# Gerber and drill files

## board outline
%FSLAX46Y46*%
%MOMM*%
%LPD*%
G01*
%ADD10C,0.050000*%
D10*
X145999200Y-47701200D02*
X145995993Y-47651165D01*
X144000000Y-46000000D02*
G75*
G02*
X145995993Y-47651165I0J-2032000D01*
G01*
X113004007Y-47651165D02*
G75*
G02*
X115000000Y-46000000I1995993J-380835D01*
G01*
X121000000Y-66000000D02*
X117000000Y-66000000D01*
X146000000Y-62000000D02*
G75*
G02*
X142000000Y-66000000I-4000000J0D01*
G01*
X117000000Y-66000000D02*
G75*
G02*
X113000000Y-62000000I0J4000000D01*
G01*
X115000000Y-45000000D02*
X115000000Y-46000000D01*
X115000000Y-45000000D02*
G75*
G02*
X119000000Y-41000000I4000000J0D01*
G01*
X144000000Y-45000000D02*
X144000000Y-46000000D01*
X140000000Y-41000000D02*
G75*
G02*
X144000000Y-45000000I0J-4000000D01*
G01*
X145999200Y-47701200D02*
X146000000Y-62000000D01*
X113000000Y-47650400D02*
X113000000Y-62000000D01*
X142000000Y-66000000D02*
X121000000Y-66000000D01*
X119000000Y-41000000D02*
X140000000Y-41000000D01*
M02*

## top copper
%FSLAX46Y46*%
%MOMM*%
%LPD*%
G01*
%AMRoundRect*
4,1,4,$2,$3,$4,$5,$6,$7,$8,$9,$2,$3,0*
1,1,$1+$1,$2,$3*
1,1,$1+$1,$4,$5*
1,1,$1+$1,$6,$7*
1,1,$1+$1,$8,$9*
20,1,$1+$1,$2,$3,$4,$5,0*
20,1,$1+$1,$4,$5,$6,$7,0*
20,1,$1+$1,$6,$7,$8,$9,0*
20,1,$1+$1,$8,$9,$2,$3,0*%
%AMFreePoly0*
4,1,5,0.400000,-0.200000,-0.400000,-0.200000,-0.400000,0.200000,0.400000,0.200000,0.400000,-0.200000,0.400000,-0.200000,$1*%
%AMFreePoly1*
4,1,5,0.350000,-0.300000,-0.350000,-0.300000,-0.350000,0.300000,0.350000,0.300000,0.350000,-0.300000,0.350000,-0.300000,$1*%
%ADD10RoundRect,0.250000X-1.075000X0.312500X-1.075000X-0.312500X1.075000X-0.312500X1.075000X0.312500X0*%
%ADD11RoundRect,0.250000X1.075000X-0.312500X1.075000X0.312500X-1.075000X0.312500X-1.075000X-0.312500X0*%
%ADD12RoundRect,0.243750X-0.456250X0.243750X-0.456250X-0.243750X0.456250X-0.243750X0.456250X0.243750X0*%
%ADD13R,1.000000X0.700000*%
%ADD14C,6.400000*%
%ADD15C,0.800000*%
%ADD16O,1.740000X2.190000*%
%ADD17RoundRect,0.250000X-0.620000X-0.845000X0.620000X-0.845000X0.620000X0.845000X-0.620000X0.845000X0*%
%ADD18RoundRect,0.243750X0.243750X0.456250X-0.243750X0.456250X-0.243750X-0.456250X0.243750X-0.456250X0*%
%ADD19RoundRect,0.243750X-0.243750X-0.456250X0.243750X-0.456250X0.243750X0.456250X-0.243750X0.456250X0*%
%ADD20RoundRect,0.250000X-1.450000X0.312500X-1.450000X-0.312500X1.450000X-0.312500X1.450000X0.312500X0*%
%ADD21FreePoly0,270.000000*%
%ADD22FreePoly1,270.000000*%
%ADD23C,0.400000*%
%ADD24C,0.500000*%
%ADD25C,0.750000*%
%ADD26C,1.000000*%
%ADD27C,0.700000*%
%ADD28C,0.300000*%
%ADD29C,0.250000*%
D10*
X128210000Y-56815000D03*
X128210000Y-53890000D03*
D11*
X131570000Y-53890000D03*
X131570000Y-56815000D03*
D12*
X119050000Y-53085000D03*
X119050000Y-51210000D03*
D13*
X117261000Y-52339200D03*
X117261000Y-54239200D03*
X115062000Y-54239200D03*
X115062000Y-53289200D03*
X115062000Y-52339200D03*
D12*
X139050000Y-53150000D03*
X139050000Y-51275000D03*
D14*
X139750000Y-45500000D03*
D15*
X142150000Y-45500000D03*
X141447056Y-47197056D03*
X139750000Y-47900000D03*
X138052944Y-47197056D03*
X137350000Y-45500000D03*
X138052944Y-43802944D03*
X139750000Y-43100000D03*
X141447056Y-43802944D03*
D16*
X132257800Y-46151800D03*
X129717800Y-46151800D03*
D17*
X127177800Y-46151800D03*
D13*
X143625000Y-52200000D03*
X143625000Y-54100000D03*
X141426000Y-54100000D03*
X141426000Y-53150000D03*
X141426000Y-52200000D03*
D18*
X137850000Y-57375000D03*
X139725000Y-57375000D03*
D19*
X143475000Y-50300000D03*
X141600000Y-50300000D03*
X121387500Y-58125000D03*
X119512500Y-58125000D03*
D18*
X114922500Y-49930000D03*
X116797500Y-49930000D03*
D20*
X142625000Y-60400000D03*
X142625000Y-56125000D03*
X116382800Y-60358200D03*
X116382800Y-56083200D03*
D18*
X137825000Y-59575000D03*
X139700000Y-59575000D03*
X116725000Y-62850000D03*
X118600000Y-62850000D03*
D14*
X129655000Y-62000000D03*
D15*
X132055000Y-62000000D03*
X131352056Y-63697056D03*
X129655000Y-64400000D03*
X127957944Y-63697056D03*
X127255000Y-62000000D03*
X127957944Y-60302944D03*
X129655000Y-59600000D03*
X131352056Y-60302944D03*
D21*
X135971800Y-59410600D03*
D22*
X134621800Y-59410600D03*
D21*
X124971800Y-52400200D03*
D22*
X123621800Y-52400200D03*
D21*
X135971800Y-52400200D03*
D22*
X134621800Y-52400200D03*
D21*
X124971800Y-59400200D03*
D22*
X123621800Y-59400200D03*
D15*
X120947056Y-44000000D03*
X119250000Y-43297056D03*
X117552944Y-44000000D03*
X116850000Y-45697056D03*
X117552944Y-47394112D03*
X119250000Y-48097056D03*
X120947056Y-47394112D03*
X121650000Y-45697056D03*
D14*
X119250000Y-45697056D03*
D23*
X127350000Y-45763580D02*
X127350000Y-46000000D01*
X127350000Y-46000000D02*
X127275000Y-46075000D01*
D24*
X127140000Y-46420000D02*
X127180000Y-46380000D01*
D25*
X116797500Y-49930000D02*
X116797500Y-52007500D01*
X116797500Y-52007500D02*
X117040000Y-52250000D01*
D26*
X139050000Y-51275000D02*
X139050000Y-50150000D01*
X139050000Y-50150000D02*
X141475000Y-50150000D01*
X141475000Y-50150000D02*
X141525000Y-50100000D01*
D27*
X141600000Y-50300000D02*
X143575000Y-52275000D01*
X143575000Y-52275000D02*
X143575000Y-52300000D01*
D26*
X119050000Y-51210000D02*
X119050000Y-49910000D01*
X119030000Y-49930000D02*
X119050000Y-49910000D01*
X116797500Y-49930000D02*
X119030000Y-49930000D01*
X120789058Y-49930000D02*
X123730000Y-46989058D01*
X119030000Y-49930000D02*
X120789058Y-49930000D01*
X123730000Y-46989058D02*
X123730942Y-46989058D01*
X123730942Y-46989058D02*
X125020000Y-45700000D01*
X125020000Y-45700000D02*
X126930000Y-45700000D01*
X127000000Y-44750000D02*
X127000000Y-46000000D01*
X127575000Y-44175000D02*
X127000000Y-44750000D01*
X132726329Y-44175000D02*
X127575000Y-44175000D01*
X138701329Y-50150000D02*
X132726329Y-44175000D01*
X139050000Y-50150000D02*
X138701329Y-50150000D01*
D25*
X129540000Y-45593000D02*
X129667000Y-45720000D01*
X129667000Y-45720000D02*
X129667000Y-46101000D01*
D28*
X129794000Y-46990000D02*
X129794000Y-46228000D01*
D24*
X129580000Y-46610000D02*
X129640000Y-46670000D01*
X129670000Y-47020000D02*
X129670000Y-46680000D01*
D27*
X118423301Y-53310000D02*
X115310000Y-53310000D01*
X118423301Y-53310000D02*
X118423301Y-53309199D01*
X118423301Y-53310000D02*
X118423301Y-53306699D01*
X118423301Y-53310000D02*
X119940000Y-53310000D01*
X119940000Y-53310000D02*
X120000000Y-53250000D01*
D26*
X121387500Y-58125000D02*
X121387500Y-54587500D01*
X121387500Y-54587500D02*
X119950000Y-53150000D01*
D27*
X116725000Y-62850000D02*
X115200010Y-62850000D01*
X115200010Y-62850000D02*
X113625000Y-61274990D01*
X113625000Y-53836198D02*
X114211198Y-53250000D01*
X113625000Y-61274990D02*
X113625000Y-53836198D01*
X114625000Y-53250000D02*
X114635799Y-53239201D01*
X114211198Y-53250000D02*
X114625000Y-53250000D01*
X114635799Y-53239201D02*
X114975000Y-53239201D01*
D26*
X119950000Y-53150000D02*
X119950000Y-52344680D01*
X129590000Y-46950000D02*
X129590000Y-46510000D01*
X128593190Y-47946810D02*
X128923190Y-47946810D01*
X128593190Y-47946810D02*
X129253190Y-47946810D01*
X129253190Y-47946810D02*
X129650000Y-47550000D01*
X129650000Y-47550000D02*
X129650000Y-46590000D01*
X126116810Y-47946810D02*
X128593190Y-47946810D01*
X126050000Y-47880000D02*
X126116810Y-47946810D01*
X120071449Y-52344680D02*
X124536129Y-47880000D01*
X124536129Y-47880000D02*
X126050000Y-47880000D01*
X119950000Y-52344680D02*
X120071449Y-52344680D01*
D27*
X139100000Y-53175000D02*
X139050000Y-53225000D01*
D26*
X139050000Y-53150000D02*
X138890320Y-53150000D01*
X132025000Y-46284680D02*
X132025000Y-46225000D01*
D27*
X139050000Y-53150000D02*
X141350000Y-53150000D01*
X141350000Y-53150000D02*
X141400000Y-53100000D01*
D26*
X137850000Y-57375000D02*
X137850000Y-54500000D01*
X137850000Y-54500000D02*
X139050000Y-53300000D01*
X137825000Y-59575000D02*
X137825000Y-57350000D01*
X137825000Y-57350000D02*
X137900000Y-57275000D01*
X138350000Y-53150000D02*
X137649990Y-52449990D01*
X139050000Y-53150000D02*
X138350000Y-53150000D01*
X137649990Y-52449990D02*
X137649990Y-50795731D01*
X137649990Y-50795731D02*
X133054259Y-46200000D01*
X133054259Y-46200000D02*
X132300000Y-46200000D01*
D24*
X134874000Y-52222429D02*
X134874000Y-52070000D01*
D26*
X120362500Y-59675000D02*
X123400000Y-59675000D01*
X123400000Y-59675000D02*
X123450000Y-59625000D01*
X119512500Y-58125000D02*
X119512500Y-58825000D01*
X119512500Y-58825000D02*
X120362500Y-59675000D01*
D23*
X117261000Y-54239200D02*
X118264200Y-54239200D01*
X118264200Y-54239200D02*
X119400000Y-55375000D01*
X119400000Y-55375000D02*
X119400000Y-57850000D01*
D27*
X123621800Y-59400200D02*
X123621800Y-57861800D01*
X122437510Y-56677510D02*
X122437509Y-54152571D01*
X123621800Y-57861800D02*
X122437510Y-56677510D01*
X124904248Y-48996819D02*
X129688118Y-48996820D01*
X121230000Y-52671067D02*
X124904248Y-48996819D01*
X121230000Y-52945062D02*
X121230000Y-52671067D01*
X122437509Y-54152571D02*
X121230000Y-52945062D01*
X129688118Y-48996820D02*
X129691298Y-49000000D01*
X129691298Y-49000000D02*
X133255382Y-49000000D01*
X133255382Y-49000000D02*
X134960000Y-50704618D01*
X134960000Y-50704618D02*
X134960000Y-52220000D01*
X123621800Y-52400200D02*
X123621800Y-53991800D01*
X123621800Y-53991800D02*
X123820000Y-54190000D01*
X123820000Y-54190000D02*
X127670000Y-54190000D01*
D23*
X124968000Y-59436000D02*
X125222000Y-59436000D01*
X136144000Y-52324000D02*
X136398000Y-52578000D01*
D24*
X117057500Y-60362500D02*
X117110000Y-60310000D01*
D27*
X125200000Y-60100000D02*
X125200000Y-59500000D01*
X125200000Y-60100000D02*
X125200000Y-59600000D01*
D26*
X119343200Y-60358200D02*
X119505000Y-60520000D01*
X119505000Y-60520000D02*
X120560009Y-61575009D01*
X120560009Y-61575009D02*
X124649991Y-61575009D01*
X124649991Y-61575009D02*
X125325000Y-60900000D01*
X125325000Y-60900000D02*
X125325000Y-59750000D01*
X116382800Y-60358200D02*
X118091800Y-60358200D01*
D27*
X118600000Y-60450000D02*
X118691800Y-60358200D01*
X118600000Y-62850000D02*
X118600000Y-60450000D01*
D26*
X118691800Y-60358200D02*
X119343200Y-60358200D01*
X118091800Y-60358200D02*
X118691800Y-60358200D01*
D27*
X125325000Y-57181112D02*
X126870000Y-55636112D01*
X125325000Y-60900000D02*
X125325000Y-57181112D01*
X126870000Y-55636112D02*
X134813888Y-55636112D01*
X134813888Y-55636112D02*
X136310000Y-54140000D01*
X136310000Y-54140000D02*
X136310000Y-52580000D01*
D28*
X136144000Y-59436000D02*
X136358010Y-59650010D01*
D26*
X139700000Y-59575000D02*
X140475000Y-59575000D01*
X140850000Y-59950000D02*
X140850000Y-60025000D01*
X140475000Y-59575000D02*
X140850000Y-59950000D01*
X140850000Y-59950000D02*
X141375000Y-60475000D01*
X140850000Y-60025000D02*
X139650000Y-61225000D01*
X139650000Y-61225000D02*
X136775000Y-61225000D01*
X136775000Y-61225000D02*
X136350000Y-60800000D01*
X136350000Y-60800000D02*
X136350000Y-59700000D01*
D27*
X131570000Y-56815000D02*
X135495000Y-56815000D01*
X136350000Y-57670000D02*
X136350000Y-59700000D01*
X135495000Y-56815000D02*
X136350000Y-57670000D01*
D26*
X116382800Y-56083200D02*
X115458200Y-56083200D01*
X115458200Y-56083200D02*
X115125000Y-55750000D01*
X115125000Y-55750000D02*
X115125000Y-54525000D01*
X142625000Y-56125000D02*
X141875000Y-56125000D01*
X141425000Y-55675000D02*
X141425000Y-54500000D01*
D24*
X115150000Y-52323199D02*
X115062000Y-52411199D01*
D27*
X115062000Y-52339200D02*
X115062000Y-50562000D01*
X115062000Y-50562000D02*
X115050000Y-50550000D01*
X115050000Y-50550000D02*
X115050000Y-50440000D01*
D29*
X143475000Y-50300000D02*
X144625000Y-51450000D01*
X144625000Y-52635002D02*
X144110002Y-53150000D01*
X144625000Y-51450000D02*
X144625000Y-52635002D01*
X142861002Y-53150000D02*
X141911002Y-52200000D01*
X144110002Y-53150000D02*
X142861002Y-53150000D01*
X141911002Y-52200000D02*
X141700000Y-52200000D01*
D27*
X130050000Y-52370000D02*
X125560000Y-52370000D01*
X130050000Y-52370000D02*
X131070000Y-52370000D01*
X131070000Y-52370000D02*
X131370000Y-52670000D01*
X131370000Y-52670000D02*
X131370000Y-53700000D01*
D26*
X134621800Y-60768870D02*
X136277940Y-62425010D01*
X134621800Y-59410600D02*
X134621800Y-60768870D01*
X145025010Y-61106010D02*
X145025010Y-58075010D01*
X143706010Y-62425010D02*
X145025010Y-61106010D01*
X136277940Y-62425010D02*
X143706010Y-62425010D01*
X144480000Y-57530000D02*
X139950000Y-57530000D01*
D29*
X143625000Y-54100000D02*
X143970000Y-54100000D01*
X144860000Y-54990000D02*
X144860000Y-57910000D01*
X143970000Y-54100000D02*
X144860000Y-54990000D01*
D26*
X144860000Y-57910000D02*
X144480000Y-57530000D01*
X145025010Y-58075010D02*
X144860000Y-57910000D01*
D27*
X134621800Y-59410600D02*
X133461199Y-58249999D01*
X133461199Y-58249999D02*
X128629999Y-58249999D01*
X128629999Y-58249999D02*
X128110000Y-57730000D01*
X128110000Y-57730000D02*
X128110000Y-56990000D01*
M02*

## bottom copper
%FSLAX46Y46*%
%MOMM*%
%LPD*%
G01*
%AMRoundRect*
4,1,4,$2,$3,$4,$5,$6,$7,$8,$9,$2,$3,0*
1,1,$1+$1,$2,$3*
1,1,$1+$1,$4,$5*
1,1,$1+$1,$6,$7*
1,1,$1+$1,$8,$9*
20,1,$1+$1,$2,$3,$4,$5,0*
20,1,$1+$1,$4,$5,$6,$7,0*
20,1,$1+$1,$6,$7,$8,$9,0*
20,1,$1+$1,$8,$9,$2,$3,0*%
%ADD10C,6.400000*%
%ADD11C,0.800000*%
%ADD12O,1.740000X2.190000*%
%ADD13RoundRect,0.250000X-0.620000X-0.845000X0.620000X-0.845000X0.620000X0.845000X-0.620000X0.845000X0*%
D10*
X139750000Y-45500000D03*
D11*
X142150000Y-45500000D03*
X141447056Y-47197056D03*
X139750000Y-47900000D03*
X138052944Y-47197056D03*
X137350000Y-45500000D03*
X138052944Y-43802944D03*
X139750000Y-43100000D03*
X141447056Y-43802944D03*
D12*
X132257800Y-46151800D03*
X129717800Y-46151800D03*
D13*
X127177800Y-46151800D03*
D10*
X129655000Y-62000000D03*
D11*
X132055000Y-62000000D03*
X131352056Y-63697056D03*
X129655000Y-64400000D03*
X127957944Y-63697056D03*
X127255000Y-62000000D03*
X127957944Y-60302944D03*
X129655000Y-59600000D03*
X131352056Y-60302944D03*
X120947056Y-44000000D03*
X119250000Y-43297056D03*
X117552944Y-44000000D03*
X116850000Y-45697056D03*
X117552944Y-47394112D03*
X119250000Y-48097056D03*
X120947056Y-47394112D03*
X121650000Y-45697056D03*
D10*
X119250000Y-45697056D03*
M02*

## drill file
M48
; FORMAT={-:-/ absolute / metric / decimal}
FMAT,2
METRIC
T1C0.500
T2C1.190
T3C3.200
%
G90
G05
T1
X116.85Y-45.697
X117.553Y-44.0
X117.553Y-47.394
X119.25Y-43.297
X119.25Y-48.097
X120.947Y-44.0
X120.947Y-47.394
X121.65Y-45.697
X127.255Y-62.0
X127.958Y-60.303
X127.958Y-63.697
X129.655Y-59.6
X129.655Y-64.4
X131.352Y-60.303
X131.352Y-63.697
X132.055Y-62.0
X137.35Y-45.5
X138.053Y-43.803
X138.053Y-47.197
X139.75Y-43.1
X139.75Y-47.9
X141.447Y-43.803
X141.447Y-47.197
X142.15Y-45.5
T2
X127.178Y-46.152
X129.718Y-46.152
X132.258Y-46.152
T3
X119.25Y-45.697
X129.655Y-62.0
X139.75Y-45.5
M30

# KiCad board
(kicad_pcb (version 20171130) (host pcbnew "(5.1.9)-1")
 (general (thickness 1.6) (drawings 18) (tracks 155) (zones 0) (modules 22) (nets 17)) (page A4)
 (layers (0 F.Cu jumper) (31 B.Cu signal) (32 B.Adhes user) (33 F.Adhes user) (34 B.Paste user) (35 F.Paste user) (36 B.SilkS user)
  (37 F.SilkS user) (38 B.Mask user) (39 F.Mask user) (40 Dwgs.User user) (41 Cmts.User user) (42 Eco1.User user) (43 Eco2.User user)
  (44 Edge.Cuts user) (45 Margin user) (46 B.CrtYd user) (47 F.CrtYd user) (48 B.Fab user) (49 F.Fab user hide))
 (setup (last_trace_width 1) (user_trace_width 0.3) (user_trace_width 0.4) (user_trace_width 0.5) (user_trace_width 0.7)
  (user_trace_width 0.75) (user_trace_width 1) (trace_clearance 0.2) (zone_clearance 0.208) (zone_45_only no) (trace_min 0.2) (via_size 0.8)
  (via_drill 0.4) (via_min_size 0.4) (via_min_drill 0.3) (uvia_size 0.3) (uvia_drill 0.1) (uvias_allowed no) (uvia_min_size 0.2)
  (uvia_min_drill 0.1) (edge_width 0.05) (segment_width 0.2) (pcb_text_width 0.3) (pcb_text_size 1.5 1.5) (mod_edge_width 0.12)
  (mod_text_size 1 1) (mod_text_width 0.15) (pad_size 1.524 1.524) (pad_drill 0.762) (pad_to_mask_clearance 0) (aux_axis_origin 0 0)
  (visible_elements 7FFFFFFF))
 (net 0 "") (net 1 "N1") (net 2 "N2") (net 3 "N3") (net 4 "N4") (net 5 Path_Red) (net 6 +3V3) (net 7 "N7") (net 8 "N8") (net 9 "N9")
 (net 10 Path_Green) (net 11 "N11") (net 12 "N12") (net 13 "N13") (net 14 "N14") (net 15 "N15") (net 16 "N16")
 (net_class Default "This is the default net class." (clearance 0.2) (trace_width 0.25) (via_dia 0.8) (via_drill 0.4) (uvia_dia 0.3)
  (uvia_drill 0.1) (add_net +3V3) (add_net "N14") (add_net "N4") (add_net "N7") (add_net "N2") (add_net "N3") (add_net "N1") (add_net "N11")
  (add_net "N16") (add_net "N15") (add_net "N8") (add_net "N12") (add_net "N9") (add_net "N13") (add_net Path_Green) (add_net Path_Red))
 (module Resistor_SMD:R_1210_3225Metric (layer F.Cu) (at 128.21 55.3525 270)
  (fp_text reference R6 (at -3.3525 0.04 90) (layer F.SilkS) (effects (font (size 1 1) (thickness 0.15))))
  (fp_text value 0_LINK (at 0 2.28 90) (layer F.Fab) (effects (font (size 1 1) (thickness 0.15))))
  (pad 2 smd roundrect (at 1.4625 0 270) (size 1.125 2.65) (layers F.Cu F.Paste F.Mask) (roundrect_rratio 0.222222) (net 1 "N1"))
  (pad 1 smd roundrect (at -1.4625 0 270) (size 1.125 2.65) (layers F.Cu F.Paste F.Mask) (roundrect_rratio 0.222222) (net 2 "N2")))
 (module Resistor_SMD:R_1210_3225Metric (layer F.Cu) (at 131.57 55.3525 90)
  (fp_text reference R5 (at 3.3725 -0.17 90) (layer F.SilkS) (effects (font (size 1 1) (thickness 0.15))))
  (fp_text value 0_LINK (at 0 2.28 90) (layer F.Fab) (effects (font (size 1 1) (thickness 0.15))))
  (pad 2 smd roundrect (at 1.4625 0 90) (size 1.125 2.65) (layers F.Cu F.Paste F.Mask) (roundrect_rratio 0.222222) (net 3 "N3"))
  (pad 1 smd roundrect (at -1.4625 0 90) (size 1.125 2.65) (layers F.Cu F.Paste F.Mask) (roundrect_rratio 0.222222) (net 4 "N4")))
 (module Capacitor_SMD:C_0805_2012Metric (layer F.Cu) (at 119.05 52.1475 270)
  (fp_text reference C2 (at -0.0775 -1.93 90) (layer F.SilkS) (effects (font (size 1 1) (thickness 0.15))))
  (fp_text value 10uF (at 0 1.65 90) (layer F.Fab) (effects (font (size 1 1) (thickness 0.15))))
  (pad 2 smd roundrect (at 0.9375 0 270) (size 0.975 1.4) (layers F.Cu F.Paste F.Mask) (roundrect_rratio 0.25) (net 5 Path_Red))
  (pad 1 smd roundrect (at -0.9375 0 270) (size 0.975 1.4) (layers F.Cu F.Paste F.Mask) (roundrect_rratio 0.25) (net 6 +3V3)))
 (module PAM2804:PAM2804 (layer F.Cu) (at 115.062 52.3392)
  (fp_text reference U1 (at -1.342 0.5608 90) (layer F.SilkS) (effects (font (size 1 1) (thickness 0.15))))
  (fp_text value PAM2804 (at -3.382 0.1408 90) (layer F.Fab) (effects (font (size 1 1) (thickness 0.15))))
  (pad 5 smd rect (at 2.199 0) (size 1 0.7) (layers F.Cu F.Paste F.Mask) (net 6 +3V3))
  (pad 4 smd rect (at 2.199 1.9) (size 1 0.7) (layers F.Cu F.Paste F.Mask) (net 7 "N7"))
  (pad 3 smd rect (at 0 1.9) (size 1 0.7) (layers F.Cu F.Paste F.Mask) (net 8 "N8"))
  (pad 2 smd rect (at 0 0.95) (size 1 0.7) (layers F.Cu F.Paste F.Mask) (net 5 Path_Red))
  (pad 1 smd rect (at 0 0) (size 1 0.7) (layers F.Cu F.Paste F.Mask) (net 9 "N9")))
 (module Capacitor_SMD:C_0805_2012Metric (layer F.Cu) (at 139.05 52.2125 270)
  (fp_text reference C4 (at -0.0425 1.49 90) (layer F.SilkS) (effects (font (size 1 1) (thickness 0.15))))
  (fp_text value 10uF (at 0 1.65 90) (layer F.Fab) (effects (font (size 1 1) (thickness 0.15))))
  (pad 2 smd roundrect (at 0.9375 0 270) (size 0.975 1.4) (layers F.Cu F.Paste F.Mask) (roundrect_rratio 0.25) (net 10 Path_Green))
  (pad 1 smd roundrect (at -0.9375 0 270) (size 0.975 1.4) (layers F.Cu F.Paste F.Mask) (roundrect_rratio 0.25) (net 6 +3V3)))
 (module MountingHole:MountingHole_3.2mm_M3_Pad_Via (layer F.Cu) (at 139.75 45.5)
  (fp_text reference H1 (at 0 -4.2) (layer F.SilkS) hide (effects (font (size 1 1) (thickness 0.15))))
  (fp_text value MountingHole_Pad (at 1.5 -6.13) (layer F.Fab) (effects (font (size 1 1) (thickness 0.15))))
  (pad 1 thru_hole circle (at 0 0) (size 6.4 6.4) (drill 3.2) (layers *.Cu *.Mask) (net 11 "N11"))
  (pad 1 thru_hole circle (at 2.4 0) (size 0.8 0.8) (drill 0.5) (layers *.Cu *.Mask) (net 11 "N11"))
  (pad 1 thru_hole circle (at 1.697056 1.697056) (size 0.8 0.8) (drill 0.5) (layers *.Cu *.Mask) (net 11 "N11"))
  (pad 1 thru_hole circle (at 0 2.4) (size 0.8 0.8) (drill 0.5) (layers *.Cu *.Mask) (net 11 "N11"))
  (pad 1 thru_hole circle (at -1.697056 1.697056) (size 0.8 0.8) (drill 0.5) (layers *.Cu *.Mask) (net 11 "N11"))
  (pad 1 thru_hole circle (at -2.4 0) (size 0.8 0.8) (drill 0.5) (layers *.Cu *.Mask) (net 11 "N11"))
  (pad 1 thru_hole circle (at -1.697056 -1.697056) (size 0.8 0.8) (drill 0.5) (layers *.Cu *.Mask) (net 11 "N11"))
  (pad 1 thru_hole circle (at 0 -2.4) (size 0.8 0.8) (drill 0.5) (layers *.Cu *.Mask) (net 11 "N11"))
  (pad 1 thru_hole circle (at 1.697056 -1.697056) (size 0.8 0.8) (drill 0.5) (layers *.Cu *.Mask) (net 11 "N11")))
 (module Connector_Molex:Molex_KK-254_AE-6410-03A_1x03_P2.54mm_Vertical (layer F.Cu) (at 127.1778 46.1518)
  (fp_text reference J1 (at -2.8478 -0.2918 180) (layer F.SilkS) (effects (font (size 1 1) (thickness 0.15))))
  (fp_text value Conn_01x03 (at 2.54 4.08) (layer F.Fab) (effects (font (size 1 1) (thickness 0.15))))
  (pad 3 thru_hole oval (at 5.08 0) (size 1.74 2.19) (drill 1.19) (layers *.Cu *.Mask) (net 10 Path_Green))
  (pad 2 thru_hole oval (at 2.54 0) (size 1.74 2.19) (drill 1.19) (layers *.Cu *.Mask) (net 5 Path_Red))
  (pad 1 thru_hole roundrect (at 0 0) (size 1.74 2.19) (drill 1.19) (layers *.Cu *.Mask) (roundrect_rratio 0.143678) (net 6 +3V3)))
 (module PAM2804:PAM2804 (layer F.Cu) (at 141.426 52.2)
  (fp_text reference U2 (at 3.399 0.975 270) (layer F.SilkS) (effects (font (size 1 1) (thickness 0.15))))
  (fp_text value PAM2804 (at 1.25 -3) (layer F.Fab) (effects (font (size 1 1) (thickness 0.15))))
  (pad 5 smd rect (at 2.199 0) (size 1 0.7) (layers F.Cu F.Paste F.Mask) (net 6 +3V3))
  (pad 4 smd rect (at 2.199 1.9) (size 1 0.7) (layers F.Cu F.Paste F.Mask) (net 1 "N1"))
  (pad 3 smd rect (at 0 1.9) (size 1 0.7) (layers F.Cu F.Paste F.Mask) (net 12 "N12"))
  (pad 2 smd rect (at 0 0.95) (size 1 0.7) (layers F.Cu F.Paste F.Mask) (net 10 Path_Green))
  (pad 1 smd rect (at 0 0) (size 1 0.7) (layers F.Cu F.Paste F.Mask) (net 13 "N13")))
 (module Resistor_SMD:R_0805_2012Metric (layer F.Cu) (at 138.7875 57.375 180)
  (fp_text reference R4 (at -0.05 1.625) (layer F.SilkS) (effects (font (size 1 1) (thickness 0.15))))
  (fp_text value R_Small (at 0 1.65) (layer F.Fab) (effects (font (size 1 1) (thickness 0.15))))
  (pad 2 smd roundrect (at 0.9375 0 180) (size 0.975 1.4) (layers F.Cu F.Paste F.Mask) (roundrect_rratio 0.25) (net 10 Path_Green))
  (pad 1 smd roundrect (at -0.9375 0 180) (size 0.975 1.4) (layers F.Cu F.Paste F.Mask) (roundrect_rratio 0.25) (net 1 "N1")))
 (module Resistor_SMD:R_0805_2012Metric (layer F.Cu) (at 142.5375 50.3)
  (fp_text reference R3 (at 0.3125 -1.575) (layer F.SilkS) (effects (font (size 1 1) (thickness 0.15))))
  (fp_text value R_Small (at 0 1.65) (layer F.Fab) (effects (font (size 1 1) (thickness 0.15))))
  (pad 2 smd roundrect (at 0.9375 0) (size 0.975 1.4) (layers F.Cu F.Paste F.Mask) (roundrect_rratio 0.25) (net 13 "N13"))
  (pad 1 smd roundrect (at -0.9375 0) (size 0.975 1.4) (layers F.Cu F.Paste F.Mask) (roundrect_rratio 0.25) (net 6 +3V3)))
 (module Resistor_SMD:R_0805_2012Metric (layer F.Cu) (at 120.45 58.125)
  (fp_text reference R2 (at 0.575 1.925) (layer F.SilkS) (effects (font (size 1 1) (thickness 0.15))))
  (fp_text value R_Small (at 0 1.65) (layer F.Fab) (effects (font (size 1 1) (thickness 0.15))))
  (pad 2 smd roundrect (at 0.9375 0) (size 0.975 1.4) (layers F.Cu F.Paste F.Mask) (roundrect_rratio 0.25) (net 5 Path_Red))
  (pad 1 smd roundrect (at -0.9375 0) (size 0.975 1.4) (layers F.Cu F.Paste F.Mask) (roundrect_rratio 0.25) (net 7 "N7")))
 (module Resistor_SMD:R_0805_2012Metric (layer F.Cu) (at 115.86 49.93 180)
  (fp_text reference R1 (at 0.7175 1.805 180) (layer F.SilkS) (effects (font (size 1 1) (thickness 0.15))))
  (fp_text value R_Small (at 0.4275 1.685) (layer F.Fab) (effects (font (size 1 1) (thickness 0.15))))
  (pad 2 smd roundrect (at 0.9375 0 180) (size 0.975 1.4) (layers F.Cu F.Paste F.Mask) (roundrect_rratio 0.25) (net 9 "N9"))
  (pad 1 smd roundrect (at -0.9375 0 180) (size 0.975 1.4) (layers F.Cu F.Paste F.Mask) (roundrect_rratio 0.25) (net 6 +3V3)))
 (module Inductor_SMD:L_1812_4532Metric (layer F.Cu) (at 142.625 58.2625 270)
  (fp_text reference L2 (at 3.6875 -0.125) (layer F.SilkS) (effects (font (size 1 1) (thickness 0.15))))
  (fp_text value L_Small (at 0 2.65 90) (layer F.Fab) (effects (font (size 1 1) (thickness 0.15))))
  (pad 2 smd roundrect (at 2.1375 0 270) (size 1.125 3.4) (layers F.Cu F.Paste F.Mask) (roundrect_rratio 0.222222) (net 4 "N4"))
  (pad 1 smd roundrect (at -2.1375 0 270) (size 1.125 3.4) (layers F.Cu F.Paste F.Mask) (roundrect_rratio 0.222222) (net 12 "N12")))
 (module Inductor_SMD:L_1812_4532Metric (layer F.Cu) (at 116.3828 58.2207 270)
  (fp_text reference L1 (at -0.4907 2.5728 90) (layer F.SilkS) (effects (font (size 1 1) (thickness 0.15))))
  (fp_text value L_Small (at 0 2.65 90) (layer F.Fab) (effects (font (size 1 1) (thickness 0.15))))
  (pad 2 smd roundrect (at 2.1375 0 270) (size 1.125 3.4) (layers F.Cu F.Paste F.Mask) (roundrect_rratio 0.222222) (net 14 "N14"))
  (pad 1 smd roundrect (at -2.1375 0 270) (size 1.125 3.4) (layers F.Cu F.Paste F.Mask) (roundrect_rratio 0.222222) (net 8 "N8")))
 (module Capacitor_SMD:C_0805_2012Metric (layer F.Cu) (at 138.7625 59.575 180)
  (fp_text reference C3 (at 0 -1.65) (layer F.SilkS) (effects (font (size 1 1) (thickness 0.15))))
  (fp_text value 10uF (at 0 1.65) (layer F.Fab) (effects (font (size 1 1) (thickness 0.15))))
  (pad 2 smd roundrect (at 0.9375 0 180) (size 0.975 1.4) (layers F.Cu F.Paste F.Mask) (roundrect_rratio 0.25) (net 10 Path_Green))
  (pad 1 smd roundrect (at -0.9375 0 180) (size 0.975 1.4) (layers F.Cu F.Paste F.Mask) (roundrect_rratio 0.25) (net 4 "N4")))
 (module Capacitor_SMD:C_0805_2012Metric (layer F.Cu) (at 117.6625 62.85 180)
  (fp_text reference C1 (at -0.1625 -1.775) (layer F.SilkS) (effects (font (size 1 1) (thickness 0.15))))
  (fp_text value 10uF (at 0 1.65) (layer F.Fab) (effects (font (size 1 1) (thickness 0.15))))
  (pad 2 smd roundrect (at 0.9375 0 180) (size 0.975 1.4) (layers F.Cu F.Paste F.Mask) (roundrect_rratio 0.25) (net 5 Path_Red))
  (pad 1 smd roundrect (at -0.9375 0 180) (size 0.975 1.4) (layers F.Cu F.Paste F.Mask) (roundrect_rratio 0.25) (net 14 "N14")))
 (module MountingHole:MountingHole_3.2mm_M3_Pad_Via (layer F.Cu) (at 129.655 62)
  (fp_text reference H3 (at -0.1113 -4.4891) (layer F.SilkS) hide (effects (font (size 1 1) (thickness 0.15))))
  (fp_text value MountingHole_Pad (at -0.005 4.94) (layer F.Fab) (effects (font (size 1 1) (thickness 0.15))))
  (pad 1 thru_hole circle (at 0 0) (size 6.4 6.4) (drill 3.2) (layers *.Cu *.Mask) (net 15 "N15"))
  (pad 1 thru_hole circle (at 2.4 0) (size 0.8 0.8) (drill 0.5) (layers *.Cu *.Mask) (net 15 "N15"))
  (pad 1 thru_hole circle (at 1.697056 1.697056) (size 0.8 0.8) (drill 0.5) (layers *.Cu *.Mask) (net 15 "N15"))
  (pad 1 thru_hole circle (at 0 2.4) (size 0.8 0.8) (drill 0.5) (layers *.Cu *.Mask) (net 15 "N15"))
  (pad 1 thru_hole circle (at -1.697056 1.697056) (size 0.8 0.8) (drill 0.5) (layers *.Cu *.Mask) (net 15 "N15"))
  (pad 1 thru_hole circle (at -2.4 0) (size 0.8 0.8) (drill 0.5) (layers *.Cu *.Mask) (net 15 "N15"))
  (pad 1 thru_hole circle (at -1.697056 -1.697056) (size 0.8 0.8) (drill 0.5) (layers *.Cu *.Mask) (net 15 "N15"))
  (pad 1 thru_hole circle (at 0 -2.4) (size 0.8 0.8) (drill 0.5) (layers *.Cu *.Mask) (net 15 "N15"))
  (pad 1 thru_hole circle (at 1.697056 -1.697056) (size 0.8 0.8) (drill 0.5) (layers *.Cu *.Mask) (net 15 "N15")))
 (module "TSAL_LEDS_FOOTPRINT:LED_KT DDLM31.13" (layer F.Cu) (at 135.2468 59.3856 270)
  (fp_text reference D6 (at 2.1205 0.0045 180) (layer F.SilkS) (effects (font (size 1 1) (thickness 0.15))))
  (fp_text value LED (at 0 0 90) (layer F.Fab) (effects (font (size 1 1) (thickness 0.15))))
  (pad 2 smd custom (at 0.025 -0.725 270) (size 0.8 0.4) (layers F.Cu F.Paste F.Mask) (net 4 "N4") (zone_connect 0)
   (options (clearance outline) (anchor rect)) (primitives))
  (pad 1 smd custom (at 0.025 0.625 270) (size 0.7 0.6) (layers F.Cu F.Paste F.Mask) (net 1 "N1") (zone_connect 0)
   (options (clearance outline) (anchor rect)) (primitives)))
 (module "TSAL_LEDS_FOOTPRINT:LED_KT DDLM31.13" (layer F.Cu) (at 124.2468 52.3752 270)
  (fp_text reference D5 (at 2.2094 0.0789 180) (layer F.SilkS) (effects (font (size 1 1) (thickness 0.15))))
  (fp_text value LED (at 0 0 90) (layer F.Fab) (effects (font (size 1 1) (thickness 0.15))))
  (pad 2 smd custom (at 0.025 -0.725 270) (size 0.8 0.4) (layers F.Cu F.Paste F.Mask) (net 3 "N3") (zone_connect 0)
   (options (clearance outline) (anchor rect)) (primitives))
  (pad 1 smd custom (at 0.025 0.625 270) (size 0.7 0.6) (layers F.Cu F.Paste F.Mask) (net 2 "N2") (zone_connect 0)
   (options (clearance outline) (anchor rect)) (primitives)))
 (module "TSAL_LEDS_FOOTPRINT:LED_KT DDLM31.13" (layer F.Cu) (at 135.2468 52.3752 270)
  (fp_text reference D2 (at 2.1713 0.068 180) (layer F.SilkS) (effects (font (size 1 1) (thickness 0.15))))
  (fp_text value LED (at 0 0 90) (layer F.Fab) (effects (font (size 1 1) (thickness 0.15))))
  (pad 2 smd custom (at 0.025 -0.725 270) (size 0.8 0.4) (layers F.Cu F.Paste F.Mask) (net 14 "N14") (zone_connect 0)
   (options (clearance outline) (anchor rect)) (primitives))
  (pad 1 smd custom (at 0.025 0.625 270) (size 0.7 0.6) (layers F.Cu F.Paste F.Mask) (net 7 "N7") (zone_connect 0)
   (options (clearance outline) (anchor rect)) (primitives)))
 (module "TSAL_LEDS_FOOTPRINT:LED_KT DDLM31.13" (layer F.Cu) (at 124.2468 59.3752 270)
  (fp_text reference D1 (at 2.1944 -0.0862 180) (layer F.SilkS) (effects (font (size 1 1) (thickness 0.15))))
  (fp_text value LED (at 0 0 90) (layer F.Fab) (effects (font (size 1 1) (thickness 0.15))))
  (pad 2 smd custom (at 0.025 -0.725 270) (size 0.8 0.4) (layers F.Cu F.Paste F.Mask) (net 14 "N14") (zone_connect 0)
   (options (clearance outline) (anchor rect)) (primitives))
  (pad 1 smd custom (at 0.025 0.625 270) (size 0.7 0.6) (layers F.Cu F.Paste F.Mask) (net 7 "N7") (zone_connect 0)
   (options (clearance outline) (anchor rect)) (primitives)))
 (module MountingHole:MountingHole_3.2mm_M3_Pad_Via (layer F.Cu) (at 119.25 45.697056)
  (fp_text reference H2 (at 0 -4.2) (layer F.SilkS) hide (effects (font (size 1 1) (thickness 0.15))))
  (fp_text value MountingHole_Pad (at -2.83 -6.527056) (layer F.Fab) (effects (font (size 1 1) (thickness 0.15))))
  (pad 1 thru_hole circle (at 1.697056 -1.697056) (size 0.8 0.8) (drill 0.5) (layers *.Cu *.Mask) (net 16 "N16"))
  (pad 1 thru_hole circle (at 0 -2.4) (size 0.8 0.8) (drill 0.5) (layers *.Cu *.Mask) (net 16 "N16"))
  (pad 1 thru_hole circle (at -1.697056 -1.697056) (size 0.8 0.8) (drill 0.5) (layers *.Cu *.Mask) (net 16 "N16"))
  (pad 1 thru_hole circle (at -2.4 0) (size 0.8 0.8) (drill 0.5) (layers *.Cu *.Mask) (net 16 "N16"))
  (pad 1 thru_hole circle (at -1.697056 1.697056) (size 0.8 0.8) (drill 0.5) (layers *.Cu *.Mask) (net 16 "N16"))
  (pad 1 thru_hole circle (at 0 2.4) (size 0.8 0.8) (drill 0.5) (layers *.Cu *.Mask) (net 16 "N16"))
  (pad 1 thru_hole circle (at 1.697056 1.697056) (size 0.8 0.8) (drill 0.5) (layers *.Cu *.Mask) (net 16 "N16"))
  (pad 1 thru_hole circle (at 2.4 0) (size 0.8 0.8) (drill 0.5) (layers *.Cu *.Mask) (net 16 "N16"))
  (pad 1 thru_hole circle (at 0 0) (size 6.4 6.4) (drill 3.2) (layers *.Cu *.Mask) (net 16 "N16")))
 (gr_line (start 145.9992 47.7012) (end 145.995993 47.651165) (layer Edge.Cuts) (width 0.05))
 (gr_arc (start 144 48.032) (end 144 46) (angle 79.1978127) (layer Edge.Cuts) (width 0.05))
 (gr_arc (start 115 48.032) (end 115 46) (angle -79.1978127) (layer Edge.Cuts) (width 0.05))
 (gr_line (start 121 66) (end 117 66) (layer Edge.Cuts) (width 0.05))
 (gr_arc (start 142 62) (end 142 66) (angle -90) (layer Edge.Cuts) (width 0.05))
 (gr_arc (start 117 62) (end 113 62) (angle -90) (layer Edge.Cuts) (width 0.05))
 (gr_line (start 115 45) (end 115 46) (layer Edge.Cuts) (width 0.05))
 (gr_arc (start 119 45) (end 119 41) (angle -90) (layer Edge.Cuts) (width 0.05))
 (gr_line (start 144 45) (end 144 46) (layer Edge.Cuts) (width 0.05))
 (gr_arc (start 140 45) (end 144 45) (angle -90) (layer Edge.Cuts) (width 0.05))
 (gr_line (start 145.9992 47.7012) (end 146 62) (layer Edge.Cuts) (width 0.05))
 (gr_line (start 113 47.6504) (end 113 62) (layer Edge.Cuts) (width 0.05))
 (gr_line (start 142 66) (end 121 66) (layer Edge.Cuts) (width 0.05))
 (gr_line (start 119 41) (end 140 41) (layer Edge.Cuts) (width 0.05))
 (segment (start 127.35 45.76358) (end 127.35 46) (width 0.4) (layer F.Cu) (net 6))
 (segment (start 127.35 46) (end 127.275 46.075) (width 0.4) (layer F.Cu) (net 6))
 (segment (start 127.14 46.42) (end 127.18 46.38) (width 0.5) (layer F.Cu) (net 6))
 (segment (start 116.7975 49.93) (end 116.7975 52.0075) (width 0.75) (layer F.Cu) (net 6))
 (segment (start 116.7975 52.0075) (end 117.04 52.25) (width 0.75) (layer F.Cu) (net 6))
 (segment (start 139.05 51.275) (end 139.05 50.15) (width 1) (layer F.Cu) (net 6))
 (segment (start 139.05 50.15) (end 141.475 50.15) (width 1) (layer F.Cu) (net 6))
 (segment (start 141.475 50.15) (end 141.525 50.1) (width 1) (layer F.Cu) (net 6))
 (segment (start 141.6 50.3) (end 143.575 52.275) (width 0.7) (layer F.Cu) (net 6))
 (segment (start 143.575 52.275) (end 143.575 52.3) (width 0.7) (layer F.Cu) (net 6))
 (segment (start 119.05 51.21) (end 119.05 49.91) (width 1) (layer F.Cu) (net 6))
 (segment (start 119.03 49.93) (end 119.05 49.91) (width 1) (layer F.Cu) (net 6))
 (segment (start 116.7975 49.93) (end 119.03 49.93) (width 1) (layer F.Cu) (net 6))
 (segment (start 120.789058 49.93) (end 123.73 46.989058) (width 1) (layer F.Cu) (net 6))
 (segment (start 119.03 49.93) (end 120.789058 49.93) (width 1) (layer F.Cu) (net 6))
 (segment (start 123.73 46.989058) (end 123.730942 46.989058) (width 1) (layer F.Cu) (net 6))
 (segment (start 123.730942 46.989058) (end 125.02 45.7) (width 1) (layer F.Cu) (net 6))
 (segment (start 125.02 45.7) (end 126.93 45.7) (width 1) (layer F.Cu) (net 6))
 (segment (start 127 44.75) (end 127 46) (width 1) (layer F.Cu) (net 6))
 (segment (start 127.575 44.175) (end 127 44.75) (width 1) (layer F.Cu) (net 6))
 (segment (start 132.726329 44.175) (end 127.575 44.175) (width 1) (layer F.Cu) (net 6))
 (segment (start 138.701329 50.15) (end 132.726329 44.175) (width 1) (layer F.Cu) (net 6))
 (segment (start 139.05 50.15) (end 138.701329 50.15) (width 1) (layer F.Cu) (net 6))
 (segment (start 129.54 45.593) (end 129.667 45.72) (width 0.75) (layer F.Cu) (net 5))
 (segment (start 129.667 45.72) (end 129.667 46.101) (width 0.75) (layer F.Cu) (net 5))
 (segment (start 129.794 46.99) (end 129.794 46.228) (width 0.3) (layer F.Cu) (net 5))
 (segment (start 129.58 46.61) (end 129.64 46.67) (width 0.5) (layer F.Cu) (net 5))
 (segment (start 129.67 47.02) (end 129.67 46.68) (width 0.5) (layer F.Cu) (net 5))
 (segment (start 118.423301 53.31) (end 115.31 53.31) (width 0.7) (layer F.Cu) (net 5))
 (segment (start 118.423301 53.31) (end 118.423301 53.309199) (width 0.7) (layer F.Cu) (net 5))
 (segment (start 118.423301 53.31) (end 118.423301 53.306699) (width 0.7) (layer F.Cu) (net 5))
 (segment (start 118.423301 53.31) (end 119.94 53.31) (width 0.7) (layer F.Cu) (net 5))
 (segment (start 119.94 53.31) (end 120 53.25) (width 0.7) (layer F.Cu) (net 5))
 (segment (start 121.3875 58.125) (end 121.3875 54.5875) (width 1) (layer F.Cu) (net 5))
 (segment (start 121.3875 54.5875) (end 119.95 53.15) (width 1) (layer F.Cu) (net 5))
 (segment (start 116.725 62.85) (end 115.20001 62.85) (width 0.7) (layer F.Cu) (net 5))
 (segment (start 115.20001 62.85) (end 113.625 61.27499) (width 0.7) (layer F.Cu) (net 5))
 (segment (start 113.625 53.836198) (end 114.211198 53.25) (width 0.7) (layer F.Cu) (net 5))
 (segment (start 113.625 61.27499) (end 113.625 53.836198) (width 0.7) (layer F.Cu) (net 5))
 (segment (start 114.625 53.25) (end 114.635799 53.239201) (width 0.7) (layer F.Cu) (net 5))
 (segment (start 114.211198 53.25) (end 114.625 53.25) (width 0.7) (layer F.Cu) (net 5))
 (segment (start 114.635799 53.239201) (end 114.975 53.239201) (width 0.7) (layer F.Cu) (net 5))
 (segment (start 119.95 53.15) (end 119.95 52.34468) (width 1) (layer F.Cu) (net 5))
 (segment (start 129.59 46.95) (end 129.59 46.51) (width 1) (layer F.Cu) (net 5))
 (segment (start 128.59319 47.94681) (end 128.92319 47.94681) (width 1) (layer F.Cu) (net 5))
 (segment (start 128.59319 47.94681) (end 129.25319 47.94681) (width 1) (layer F.Cu) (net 5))
 (segment (start 129.25319 47.94681) (end 129.65 47.55) (width 1) (layer F.Cu) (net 5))
 (segment (start 129.65 47.55) (end 129.65 46.59) (width 1) (layer F.Cu) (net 5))
 (segment (start 126.11681 47.94681) (end 128.59319 47.94681) (width 1) (layer F.Cu) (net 5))
 (segment (start 126.05 47.88) (end 126.11681 47.94681) (width 1) (layer F.Cu) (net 5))
 (segment (start 120.071449 52.34468) (end 124.536129 47.88) (width 1) (layer F.Cu) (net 5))
 (segment (start 124.536129 47.88) (end 126.05 47.88) (width 1) (layer F.Cu) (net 5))
 (segment (start 119.95 52.34468) (end 120.071449 52.34468) (width 1) (layer F.Cu) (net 5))
 (segment (start 139.1 53.175) (end 139.05 53.225) (width 0.7) (layer F.Cu) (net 10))
 (segment (start 139.05 53.15) (end 138.89032 53.15) (width 1) (layer F.Cu) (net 10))
 (segment (start 132.025 46.28468) (end 132.025 46.225) (width 1) (layer F.Cu) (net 10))
 (segment (start 139.05 53.15) (end 141.35 53.15) (width 0.7) (layer F.Cu) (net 10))
 (segment (start 141.35 53.15) (end 141.4 53.1) (width 0.7) (layer F.Cu) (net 10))
 (segment (start 137.85 57.375) (end 137.85 54.5) (width 1) (layer F.Cu) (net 10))
 (segment (start 137.85 54.5) (end 139.05 53.3) (width 1) (layer F.Cu) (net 10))
 (segment (start 137.825 59.575) (end 137.825 57.35) (width 1) (layer F.Cu) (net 10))
 (segment (start 137.825 57.35) (end 137.9 57.275) (width 1) (layer F.Cu) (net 10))
 (segment (start 138.35 53.15) (end 137.64999 52.44999) (width 1) (layer F.Cu) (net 10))
 (segment (start 139.05 53.15) (end 138.35 53.15) (width 1) (layer F.Cu) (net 10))
 (segment (start 137.64999 52.44999) (end 137.64999 50.795731) (width 1) (layer F.Cu) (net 10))
 (segment (start 137.64999 50.795731) (end 133.054259 46.2) (width 1) (layer F.Cu) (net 10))
 (segment (start 133.054259 46.2) (end 132.3 46.2) (width 1) (layer F.Cu) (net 10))
 (segment (start 134.874 52.222429) (end 134.874 52.07) (width 0.5) (layer F.Cu) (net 7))
 (segment (start 120.3625 59.675) (end 123.4 59.675) (width 1) (layer F.Cu) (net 7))
 (segment (start 123.4 59.675) (end 123.45 59.625) (width 1) (layer F.Cu) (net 7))
 (segment (start 119.5125 58.125) (end 119.5125 58.825) (width 1) (layer F.Cu) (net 7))
 (segment (start 119.5125 58.825) (end 120.3625 59.675) (width 1) (layer F.Cu) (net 7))
 (segment (start 117.261 54.2392) (end 118.2642 54.2392) (width 0.4) (layer F.Cu) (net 7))
 (segment (start 118.2642 54.2392) (end 119.4 55.375) (width 0.4) (layer F.Cu) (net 7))
 (segment (start 119.4 55.375) (end 119.4 57.85) (width 0.4) (layer F.Cu) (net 7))
 (segment (start 123.6218 59.4002) (end 123.6218 57.8618) (width 0.7) (layer F.Cu) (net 7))
 (segment (start 122.43751 56.67751) (end 122.437509 54.152571) (width 0.7) (layer F.Cu) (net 7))
 (segment (start 123.6218 57.8618) (end 122.43751 56.67751) (width 0.7) (layer F.Cu) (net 7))
 (segment (start 124.904248 48.996819) (end 129.688118 48.99682) (width 0.7) (layer F.Cu) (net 7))
 (segment (start 121.23 52.671067) (end 124.904248 48.996819) (width 0.7) (layer F.Cu) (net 7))
 (segment (start 121.23 52.945062) (end 121.23 52.671067) (width 0.7) (layer F.Cu) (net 7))
 (segment (start 122.437509 54.152571) (end 121.23 52.945062) (width 0.7) (layer F.Cu) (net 7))
 (segment (start 129.688118 48.99682) (end 129.691298 49) (width 0.7) (layer F.Cu) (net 7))
 (segment (start 129.691298 49) (end 133.255382 49) (width 0.7) (layer F.Cu) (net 7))
 (segment (start 133.255382 49) (end 134.96 50.704618) (width 0.7) (layer F.Cu) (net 7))
 (segment (start 134.96 50.704618) (end 134.96 52.22) (width 0.7) (layer F.Cu) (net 7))
 (segment (start 123.6218 52.4002) (end 123.6218 53.9918) (width 0.7) (layer F.Cu) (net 2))
 (segment (start 123.6218 53.9918) (end 123.82 54.19) (width 0.7) (layer F.Cu) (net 2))
 (segment (start 123.82 54.19) (end 127.67 54.19) (width 0.7) (layer F.Cu) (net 2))
 (segment (start 124.968 59.436) (end 125.222 59.436) (width 0.4) (layer F.Cu) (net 14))
 (segment (start 136.144 52.324) (end 136.398 52.578) (width 0.4) (layer F.Cu) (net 14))
 (segment (start 117.0575 60.3625) (end 117.11 60.31) (width 0.5) (layer F.Cu) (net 14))
 (segment (start 125.2 60.1) (end 125.2 59.5) (width 0.7) (layer F.Cu) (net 14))
 (segment (start 125.2 60.1) (end 125.2 59.6) (width 0.7) (layer F.Cu) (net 14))
 (segment (start 119.3432 60.3582) (end 119.505 60.52) (width 1) (layer F.Cu) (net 14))
 (segment (start 119.505 60.52) (end 120.560009 61.575009) (width 1) (layer F.Cu) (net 14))
 (segment (start 120.560009 61.575009) (end 124.649991 61.575009) (width 1) (layer F.Cu) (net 14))
 (segment (start 124.649991 61.575009) (end 125.325 60.9) (width 1) (layer F.Cu) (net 14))
 (segment (start 125.325 60.9) (end 125.325 59.75) (width 1) (layer F.Cu) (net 14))
 (segment (start 116.3828 60.3582) (end 118.0918 60.3582) (width 1) (layer F.Cu) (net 14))
 (segment (start 118.6 60.45) (end 118.6918 60.3582) (width 0.7) (layer F.Cu) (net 14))
 (segment (start 118.6 62.85) (end 118.6 60.45) (width 0.7) (layer F.Cu) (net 14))
 (segment (start 118.6918 60.3582) (end 119.3432 60.3582) (width 1) (layer F.Cu) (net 14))
 (segment (start 118.0918 60.3582) (end 118.6918 60.3582) (width 1) (layer F.Cu) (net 14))
 (segment (start 125.325 57.181112) (end 126.87 55.636112) (width 0.7) (layer F.Cu) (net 14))
 (segment (start 125.325 60.9) (end 125.325 57.181112) (width 0.7) (layer F.Cu) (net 14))
 (segment (start 126.87 55.636112) (end 134.813888 55.636112) (width 0.7) (layer F.Cu) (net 14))
 (segment (start 134.813888 55.636112) (end 136.31 54.14) (width 0.7) (layer F.Cu) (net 14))
 (segment (start 136.31 54.14) (end 136.31 52.58) (width 0.7) (layer F.Cu) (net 14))
 (segment (start 136.144 59.436) (end 136.35801 59.65001) (width 0.3) (layer F.Cu) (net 4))
 (segment (start 139.7 59.575) (end 140.475 59.575) (width 1) (layer F.Cu) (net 4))
 (segment (start 140.85 59.95) (end 140.85 60.025) (width 1) (layer F.Cu) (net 4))
 (segment (start 140.475 59.575) (end 140.85 59.95) (width 1) (layer F.Cu) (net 4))
 (segment (start 140.85 59.95) (end 141.375 60.475) (width 1) (layer F.Cu) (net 4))
 (segment (start 140.85 60.025) (end 139.65 61.225) (width 1) (layer F.Cu) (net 4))
 (segment (start 139.65 61.225) (end 136.775 61.225) (width 1) (layer F.Cu) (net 4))
 (segment (start 136.775 61.225) (end 136.35 60.8) (width 1) (layer F.Cu) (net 4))
 (segment (start 136.35 60.8) (end 136.35 59.7) (width 1) (layer F.Cu) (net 4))
 (segment (start 131.57 56.815) (end 135.495 56.815) (width 0.7) (layer F.Cu) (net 4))
 (segment (start 136.35 57.67) (end 136.35 59.7) (width 0.7) (layer F.Cu) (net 4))
 (segment (start 135.495 56.815) (end 136.35 57.67) (width 0.7) (layer F.Cu) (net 4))
 (segment (start 116.3828 56.0832) (end 115.4582 56.0832) (width 1) (layer F.Cu) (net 8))
 (segment (start 115.4582 56.0832) (end 115.125 55.75) (width 1) (layer F.Cu) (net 8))
 (segment (start 115.125 55.75) (end 115.125 54.525) (width 1) (layer F.Cu) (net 8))
 (segment (start 142.625 56.125) (end 141.875 56.125) (width 1) (layer F.Cu) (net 12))
 (segment (start 141.425 55.675) (end 141.425 54.5) (width 1) (layer F.Cu) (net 12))
 (segment (start 115.15 52.323199) (end 115.062 52.411199) (width 0.5) (layer F.Cu) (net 9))
 (segment (start 115.062 52.3392) (end 115.062 50.562) (width 0.7) (layer F.Cu) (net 9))
 (segment (start 115.062 50.562) (end 115.05 50.55) (width 0.7) (layer F.Cu) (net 9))
 (segment (start 115.05 50.55) (end 115.05 50.44) (width 0.7) (layer F.Cu) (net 9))
 (segment (start 143.475 50.3) (end 144.625 51.45) (width 0.25) (layer F.Cu) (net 13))
 (segment (start 144.625 52.635002) (end 144.110002 53.15) (width 0.25) (layer F.Cu) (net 13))
 (segment (start 144.625 51.45) (end 144.625 52.635002) (width 0.25) (layer F.Cu) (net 13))
 (segment (start 142.861002 53.15) (end 141.911002 52.2) (width 0.25) (layer F.Cu) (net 13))
 (segment (start 144.110002 53.15) (end 142.861002 53.15) (width 0.25) (layer F.Cu) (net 13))
 (segment (start 141.911002 52.2) (end 141.7 52.2) (width 0.25) (layer F.Cu) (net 13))
 (segment (start 130.05 52.37) (end 125.56 52.37) (width 0.7) (layer F.Cu) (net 3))
 (segment (start 130.05 52.37) (end 131.07 52.37) (width 0.7) (layer F.Cu) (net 3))
 (segment (start 131.07 52.37) (end 131.37 52.67) (width 0.7) (layer F.Cu) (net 3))
 (segment (start 131.37 52.67) (end 131.37 53.7) (width 0.7) (layer F.Cu) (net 3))
 (segment (start 134.6218 60.76887) (end 136.27794 62.42501) (width 1) (layer F.Cu) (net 1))
 (segment (start 134.6218 59.4106) (end 134.6218 60.76887) (width 1) (layer F.Cu) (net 1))
 (segment (start 145.02501 61.10601) (end 145.02501 58.07501) (width 1) (layer F.Cu) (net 1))
 (segment (start 143.70601 62.42501) (end 145.02501 61.10601) (width 1) (layer F.Cu) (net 1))
 (segment (start 136.27794 62.42501) (end 143.70601 62.42501) (width 1) (layer F.Cu) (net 1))
 (segment (start 144.48 57.53) (end 139.95 57.53) (width 1) (layer F.Cu) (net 1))
 (segment (start 143.625 54.1) (end 143.97 54.1) (width 0.25) (layer F.Cu) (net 1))
 (segment (start 144.86 54.99) (end 144.86 57.91) (width 0.25) (layer F.Cu) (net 1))
 (segment (start 143.97 54.1) (end 144.86 54.99) (width 0.25) (layer F.Cu) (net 1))
 (segment (start 144.86 57.91) (end 144.48 57.53) (width 1) (layer F.Cu) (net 1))
 (segment (start 145.02501 58.07501) (end 144.86 57.91) (width 1) (layer F.Cu) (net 1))
 (segment (start 134.6218 59.4106) (end 133.461199 58.249999) (width 0.7) (layer F.Cu) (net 1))
 (segment (start 133.461199 58.249999) (end 128.629999 58.249999) (width 0.7) (layer F.Cu) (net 1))
 (segment (start 128.629999 58.249999) (end 128.11 57.73) (width 0.7) (layer F.Cu) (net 1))
 (segment (start 128.11 57.73) (end 128.11 56.99) (width 0.7) (layer F.Cu) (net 1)))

